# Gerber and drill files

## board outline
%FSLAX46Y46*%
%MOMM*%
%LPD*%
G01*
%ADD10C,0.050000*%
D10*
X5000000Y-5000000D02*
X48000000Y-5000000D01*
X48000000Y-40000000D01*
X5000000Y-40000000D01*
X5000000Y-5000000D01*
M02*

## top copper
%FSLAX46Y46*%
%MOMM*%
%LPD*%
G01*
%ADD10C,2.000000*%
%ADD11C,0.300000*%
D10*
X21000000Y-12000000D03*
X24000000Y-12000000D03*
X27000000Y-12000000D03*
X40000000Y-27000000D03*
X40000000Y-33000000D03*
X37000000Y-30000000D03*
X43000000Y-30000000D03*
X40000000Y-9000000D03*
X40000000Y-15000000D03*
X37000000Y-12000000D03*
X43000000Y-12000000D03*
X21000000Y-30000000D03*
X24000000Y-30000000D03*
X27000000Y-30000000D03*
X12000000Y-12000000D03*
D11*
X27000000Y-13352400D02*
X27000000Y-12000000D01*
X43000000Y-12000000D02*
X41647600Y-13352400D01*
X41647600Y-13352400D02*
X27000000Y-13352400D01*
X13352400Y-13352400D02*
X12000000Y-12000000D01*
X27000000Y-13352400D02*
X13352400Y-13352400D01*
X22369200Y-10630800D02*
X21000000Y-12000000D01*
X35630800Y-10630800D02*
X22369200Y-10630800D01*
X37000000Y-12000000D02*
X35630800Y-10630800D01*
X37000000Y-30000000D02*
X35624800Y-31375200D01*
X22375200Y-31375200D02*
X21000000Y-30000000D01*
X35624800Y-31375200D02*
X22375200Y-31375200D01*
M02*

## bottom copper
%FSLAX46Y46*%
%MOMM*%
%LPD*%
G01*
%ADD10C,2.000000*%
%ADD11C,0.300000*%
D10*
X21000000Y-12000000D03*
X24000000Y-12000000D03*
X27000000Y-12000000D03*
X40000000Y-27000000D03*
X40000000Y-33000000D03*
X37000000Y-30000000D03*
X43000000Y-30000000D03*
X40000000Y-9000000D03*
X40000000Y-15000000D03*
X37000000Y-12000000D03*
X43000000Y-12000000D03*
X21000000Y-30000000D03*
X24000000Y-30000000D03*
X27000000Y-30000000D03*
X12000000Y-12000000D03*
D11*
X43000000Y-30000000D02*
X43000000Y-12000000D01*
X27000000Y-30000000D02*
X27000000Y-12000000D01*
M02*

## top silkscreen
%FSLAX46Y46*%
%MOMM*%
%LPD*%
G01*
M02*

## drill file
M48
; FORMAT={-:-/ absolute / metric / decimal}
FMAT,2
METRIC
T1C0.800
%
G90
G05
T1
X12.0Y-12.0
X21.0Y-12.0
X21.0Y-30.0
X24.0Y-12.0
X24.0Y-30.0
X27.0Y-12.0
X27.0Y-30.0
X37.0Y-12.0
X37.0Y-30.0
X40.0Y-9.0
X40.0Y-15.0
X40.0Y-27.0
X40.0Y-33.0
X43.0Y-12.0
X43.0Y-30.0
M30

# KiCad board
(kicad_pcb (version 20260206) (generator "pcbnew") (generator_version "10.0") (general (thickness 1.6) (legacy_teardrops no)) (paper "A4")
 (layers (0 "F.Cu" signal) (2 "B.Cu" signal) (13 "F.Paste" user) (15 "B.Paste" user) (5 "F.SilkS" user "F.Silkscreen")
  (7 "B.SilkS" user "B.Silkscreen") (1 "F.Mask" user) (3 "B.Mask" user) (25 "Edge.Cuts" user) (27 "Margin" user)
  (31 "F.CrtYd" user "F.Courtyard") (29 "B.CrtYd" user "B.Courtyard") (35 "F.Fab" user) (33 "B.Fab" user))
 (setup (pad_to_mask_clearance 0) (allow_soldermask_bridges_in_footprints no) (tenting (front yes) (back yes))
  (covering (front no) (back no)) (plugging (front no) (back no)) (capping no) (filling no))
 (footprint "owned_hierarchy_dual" (layer "F.Cu") (at 24 12)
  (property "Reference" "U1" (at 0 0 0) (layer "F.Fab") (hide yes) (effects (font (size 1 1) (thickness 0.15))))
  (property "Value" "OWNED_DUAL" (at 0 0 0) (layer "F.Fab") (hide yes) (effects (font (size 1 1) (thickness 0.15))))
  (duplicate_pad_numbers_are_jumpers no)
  (pad "1" thru_hole circle (at -3 0) (size 2 2) (drill 0.8) (layers "*.Cu" "*.Mask") (remove_unused_layers no) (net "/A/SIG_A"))
  (pad "2" thru_hole circle (at 0 0) (size 2 2) (drill 0.8) (layers "*.Cu" "*.Mask") (remove_unused_layers no) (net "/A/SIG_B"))
  (pad "3" thru_hole circle (at 3 0) (size 2 2) (drill 0.8) (layers "*.Cu" "*.Mask") (remove_unused_layers no) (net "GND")))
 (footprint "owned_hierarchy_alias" (layer "F.Cu") (at 40 30)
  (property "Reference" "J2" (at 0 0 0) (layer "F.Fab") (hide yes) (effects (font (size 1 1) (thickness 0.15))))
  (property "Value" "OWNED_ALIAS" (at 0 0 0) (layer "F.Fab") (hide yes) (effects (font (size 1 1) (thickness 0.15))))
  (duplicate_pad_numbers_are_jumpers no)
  (pad "MP" thru_hole circle (at 0 -3) (size 2 2) (drill 0.8) (layers "*.Cu" "*.Mask") (remove_unused_layers no))
  (pad "MP" thru_hole circle (at 0 3) (size 2 2) (drill 0.8) (layers "*.Cu" "*.Mask") (remove_unused_layers no))
  (pad "R" thru_hole circle (at -3 0) (size 2 2) (drill 0.8) (layers "*.Cu" "*.Mask") (remove_unused_layers no) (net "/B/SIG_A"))
  (pad "T" thru_hole circle (at 3 0) (size 2 2) (drill 0.8) (layers "*.Cu" "*.Mask") (remove_unused_layers no) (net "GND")))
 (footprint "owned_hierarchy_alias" (layer "F.Cu") (at 40 12)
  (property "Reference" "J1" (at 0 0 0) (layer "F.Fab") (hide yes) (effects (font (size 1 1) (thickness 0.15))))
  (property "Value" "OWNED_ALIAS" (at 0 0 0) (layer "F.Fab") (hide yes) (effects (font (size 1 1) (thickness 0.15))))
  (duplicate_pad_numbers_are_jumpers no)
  (pad "MP" thru_hole circle (at 0 -3) (size 2 2) (drill 0.8) (layers "*.Cu" "*.Mask") (remove_unused_layers no))
  (pad "MP" thru_hole circle (at 0 3) (size 2 2) (drill 0.8) (layers "*.Cu" "*.Mask") (remove_unused_layers no))
  (pad "R" thru_hole circle (at -3 0) (size 2 2) (drill 0.8) (layers "*.Cu" "*.Mask") (remove_unused_layers no) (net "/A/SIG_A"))
  (pad "T" thru_hole circle (at 3 0) (size 2 2) (drill 0.8) (layers "*.Cu" "*.Mask") (remove_unused_layers no) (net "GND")))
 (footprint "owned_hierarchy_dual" (layer "F.Cu") (at 24 30)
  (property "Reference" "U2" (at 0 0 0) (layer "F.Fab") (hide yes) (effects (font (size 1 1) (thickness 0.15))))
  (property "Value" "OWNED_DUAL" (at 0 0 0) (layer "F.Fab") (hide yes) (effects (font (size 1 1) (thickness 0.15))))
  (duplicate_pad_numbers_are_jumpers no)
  (pad "1" thru_hole circle (at -3 0) (size 2 2) (drill 0.8) (layers "*.Cu" "*.Mask") (remove_unused_layers no) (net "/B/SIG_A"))
  (pad "2" thru_hole circle (at 0 0) (size 2 2) (drill 0.8) (layers "*.Cu" "*.Mask") (remove_unused_layers no) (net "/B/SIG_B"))
  (pad "3" thru_hole circle (at 3 0) (size 2 2) (drill 0.8) (layers "*.Cu" "*.Mask") (remove_unused_layers no) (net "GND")))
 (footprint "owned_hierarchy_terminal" (layer "F.Cu") (at 12 12)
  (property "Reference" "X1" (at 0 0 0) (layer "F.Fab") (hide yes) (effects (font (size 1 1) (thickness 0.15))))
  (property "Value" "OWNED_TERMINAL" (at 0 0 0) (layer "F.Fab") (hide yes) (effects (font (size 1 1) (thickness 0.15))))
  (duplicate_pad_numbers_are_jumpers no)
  (pad "1" thru_hole circle (at 0 0) (size 2 2) (drill 0.8) (layers "*.Cu" "*.Mask") (remove_unused_layers no) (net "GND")))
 (gr_rect (start 5 5) (end 48 40) (stroke (width 0.05) (type default)) (fill no) (layer "Edge.Cuts"))
 (segment (start 27 13.3524) (end 27 12) (width 0.3) (layer "F.Cu") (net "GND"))
 (segment (start 43 12) (end 41.6476 13.3524) (width 0.3) (layer "F.Cu") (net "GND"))
 (segment (start 41.6476 13.3524) (end 27 13.3524) (width 0.3) (layer "F.Cu") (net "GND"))
 (segment (start 13.3524 13.3524) (end 12 12) (width 0.3) (layer "F.Cu") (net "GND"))
 (segment (start 27 13.3524) (end 13.3524 13.3524) (width 0.3) (layer "F.Cu") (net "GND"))
 (segment (start 43 30) (end 43 12) (width 0.3) (layer "B.Cu") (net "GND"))
 (segment (start 27 30) (end 27 12) (width 0.3) (layer "B.Cu") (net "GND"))
 (segment (start 22.3692 10.6308) (end 21 12) (width 0.3) (layer "F.Cu") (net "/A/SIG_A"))
 (segment (start 35.6308 10.6308) (end 22.3692 10.6308) (width 0.3) (layer "F.Cu") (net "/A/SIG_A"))
 (segment (start 37 12) (end 35.6308 10.6308) (width 0.3) (layer "F.Cu") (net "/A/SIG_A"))
 (segment (start 37 30) (end 35.6248 31.3752) (width 0.3) (layer "F.Cu") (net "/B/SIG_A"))
 (segment (start 22.3752 31.3752) (end 21 30) (width 0.3) (layer "F.Cu") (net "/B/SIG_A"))
 (segment (start 35.6248 31.3752) (end 22.3752 31.3752) (width 0.3) (layer "F.Cu") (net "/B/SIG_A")))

